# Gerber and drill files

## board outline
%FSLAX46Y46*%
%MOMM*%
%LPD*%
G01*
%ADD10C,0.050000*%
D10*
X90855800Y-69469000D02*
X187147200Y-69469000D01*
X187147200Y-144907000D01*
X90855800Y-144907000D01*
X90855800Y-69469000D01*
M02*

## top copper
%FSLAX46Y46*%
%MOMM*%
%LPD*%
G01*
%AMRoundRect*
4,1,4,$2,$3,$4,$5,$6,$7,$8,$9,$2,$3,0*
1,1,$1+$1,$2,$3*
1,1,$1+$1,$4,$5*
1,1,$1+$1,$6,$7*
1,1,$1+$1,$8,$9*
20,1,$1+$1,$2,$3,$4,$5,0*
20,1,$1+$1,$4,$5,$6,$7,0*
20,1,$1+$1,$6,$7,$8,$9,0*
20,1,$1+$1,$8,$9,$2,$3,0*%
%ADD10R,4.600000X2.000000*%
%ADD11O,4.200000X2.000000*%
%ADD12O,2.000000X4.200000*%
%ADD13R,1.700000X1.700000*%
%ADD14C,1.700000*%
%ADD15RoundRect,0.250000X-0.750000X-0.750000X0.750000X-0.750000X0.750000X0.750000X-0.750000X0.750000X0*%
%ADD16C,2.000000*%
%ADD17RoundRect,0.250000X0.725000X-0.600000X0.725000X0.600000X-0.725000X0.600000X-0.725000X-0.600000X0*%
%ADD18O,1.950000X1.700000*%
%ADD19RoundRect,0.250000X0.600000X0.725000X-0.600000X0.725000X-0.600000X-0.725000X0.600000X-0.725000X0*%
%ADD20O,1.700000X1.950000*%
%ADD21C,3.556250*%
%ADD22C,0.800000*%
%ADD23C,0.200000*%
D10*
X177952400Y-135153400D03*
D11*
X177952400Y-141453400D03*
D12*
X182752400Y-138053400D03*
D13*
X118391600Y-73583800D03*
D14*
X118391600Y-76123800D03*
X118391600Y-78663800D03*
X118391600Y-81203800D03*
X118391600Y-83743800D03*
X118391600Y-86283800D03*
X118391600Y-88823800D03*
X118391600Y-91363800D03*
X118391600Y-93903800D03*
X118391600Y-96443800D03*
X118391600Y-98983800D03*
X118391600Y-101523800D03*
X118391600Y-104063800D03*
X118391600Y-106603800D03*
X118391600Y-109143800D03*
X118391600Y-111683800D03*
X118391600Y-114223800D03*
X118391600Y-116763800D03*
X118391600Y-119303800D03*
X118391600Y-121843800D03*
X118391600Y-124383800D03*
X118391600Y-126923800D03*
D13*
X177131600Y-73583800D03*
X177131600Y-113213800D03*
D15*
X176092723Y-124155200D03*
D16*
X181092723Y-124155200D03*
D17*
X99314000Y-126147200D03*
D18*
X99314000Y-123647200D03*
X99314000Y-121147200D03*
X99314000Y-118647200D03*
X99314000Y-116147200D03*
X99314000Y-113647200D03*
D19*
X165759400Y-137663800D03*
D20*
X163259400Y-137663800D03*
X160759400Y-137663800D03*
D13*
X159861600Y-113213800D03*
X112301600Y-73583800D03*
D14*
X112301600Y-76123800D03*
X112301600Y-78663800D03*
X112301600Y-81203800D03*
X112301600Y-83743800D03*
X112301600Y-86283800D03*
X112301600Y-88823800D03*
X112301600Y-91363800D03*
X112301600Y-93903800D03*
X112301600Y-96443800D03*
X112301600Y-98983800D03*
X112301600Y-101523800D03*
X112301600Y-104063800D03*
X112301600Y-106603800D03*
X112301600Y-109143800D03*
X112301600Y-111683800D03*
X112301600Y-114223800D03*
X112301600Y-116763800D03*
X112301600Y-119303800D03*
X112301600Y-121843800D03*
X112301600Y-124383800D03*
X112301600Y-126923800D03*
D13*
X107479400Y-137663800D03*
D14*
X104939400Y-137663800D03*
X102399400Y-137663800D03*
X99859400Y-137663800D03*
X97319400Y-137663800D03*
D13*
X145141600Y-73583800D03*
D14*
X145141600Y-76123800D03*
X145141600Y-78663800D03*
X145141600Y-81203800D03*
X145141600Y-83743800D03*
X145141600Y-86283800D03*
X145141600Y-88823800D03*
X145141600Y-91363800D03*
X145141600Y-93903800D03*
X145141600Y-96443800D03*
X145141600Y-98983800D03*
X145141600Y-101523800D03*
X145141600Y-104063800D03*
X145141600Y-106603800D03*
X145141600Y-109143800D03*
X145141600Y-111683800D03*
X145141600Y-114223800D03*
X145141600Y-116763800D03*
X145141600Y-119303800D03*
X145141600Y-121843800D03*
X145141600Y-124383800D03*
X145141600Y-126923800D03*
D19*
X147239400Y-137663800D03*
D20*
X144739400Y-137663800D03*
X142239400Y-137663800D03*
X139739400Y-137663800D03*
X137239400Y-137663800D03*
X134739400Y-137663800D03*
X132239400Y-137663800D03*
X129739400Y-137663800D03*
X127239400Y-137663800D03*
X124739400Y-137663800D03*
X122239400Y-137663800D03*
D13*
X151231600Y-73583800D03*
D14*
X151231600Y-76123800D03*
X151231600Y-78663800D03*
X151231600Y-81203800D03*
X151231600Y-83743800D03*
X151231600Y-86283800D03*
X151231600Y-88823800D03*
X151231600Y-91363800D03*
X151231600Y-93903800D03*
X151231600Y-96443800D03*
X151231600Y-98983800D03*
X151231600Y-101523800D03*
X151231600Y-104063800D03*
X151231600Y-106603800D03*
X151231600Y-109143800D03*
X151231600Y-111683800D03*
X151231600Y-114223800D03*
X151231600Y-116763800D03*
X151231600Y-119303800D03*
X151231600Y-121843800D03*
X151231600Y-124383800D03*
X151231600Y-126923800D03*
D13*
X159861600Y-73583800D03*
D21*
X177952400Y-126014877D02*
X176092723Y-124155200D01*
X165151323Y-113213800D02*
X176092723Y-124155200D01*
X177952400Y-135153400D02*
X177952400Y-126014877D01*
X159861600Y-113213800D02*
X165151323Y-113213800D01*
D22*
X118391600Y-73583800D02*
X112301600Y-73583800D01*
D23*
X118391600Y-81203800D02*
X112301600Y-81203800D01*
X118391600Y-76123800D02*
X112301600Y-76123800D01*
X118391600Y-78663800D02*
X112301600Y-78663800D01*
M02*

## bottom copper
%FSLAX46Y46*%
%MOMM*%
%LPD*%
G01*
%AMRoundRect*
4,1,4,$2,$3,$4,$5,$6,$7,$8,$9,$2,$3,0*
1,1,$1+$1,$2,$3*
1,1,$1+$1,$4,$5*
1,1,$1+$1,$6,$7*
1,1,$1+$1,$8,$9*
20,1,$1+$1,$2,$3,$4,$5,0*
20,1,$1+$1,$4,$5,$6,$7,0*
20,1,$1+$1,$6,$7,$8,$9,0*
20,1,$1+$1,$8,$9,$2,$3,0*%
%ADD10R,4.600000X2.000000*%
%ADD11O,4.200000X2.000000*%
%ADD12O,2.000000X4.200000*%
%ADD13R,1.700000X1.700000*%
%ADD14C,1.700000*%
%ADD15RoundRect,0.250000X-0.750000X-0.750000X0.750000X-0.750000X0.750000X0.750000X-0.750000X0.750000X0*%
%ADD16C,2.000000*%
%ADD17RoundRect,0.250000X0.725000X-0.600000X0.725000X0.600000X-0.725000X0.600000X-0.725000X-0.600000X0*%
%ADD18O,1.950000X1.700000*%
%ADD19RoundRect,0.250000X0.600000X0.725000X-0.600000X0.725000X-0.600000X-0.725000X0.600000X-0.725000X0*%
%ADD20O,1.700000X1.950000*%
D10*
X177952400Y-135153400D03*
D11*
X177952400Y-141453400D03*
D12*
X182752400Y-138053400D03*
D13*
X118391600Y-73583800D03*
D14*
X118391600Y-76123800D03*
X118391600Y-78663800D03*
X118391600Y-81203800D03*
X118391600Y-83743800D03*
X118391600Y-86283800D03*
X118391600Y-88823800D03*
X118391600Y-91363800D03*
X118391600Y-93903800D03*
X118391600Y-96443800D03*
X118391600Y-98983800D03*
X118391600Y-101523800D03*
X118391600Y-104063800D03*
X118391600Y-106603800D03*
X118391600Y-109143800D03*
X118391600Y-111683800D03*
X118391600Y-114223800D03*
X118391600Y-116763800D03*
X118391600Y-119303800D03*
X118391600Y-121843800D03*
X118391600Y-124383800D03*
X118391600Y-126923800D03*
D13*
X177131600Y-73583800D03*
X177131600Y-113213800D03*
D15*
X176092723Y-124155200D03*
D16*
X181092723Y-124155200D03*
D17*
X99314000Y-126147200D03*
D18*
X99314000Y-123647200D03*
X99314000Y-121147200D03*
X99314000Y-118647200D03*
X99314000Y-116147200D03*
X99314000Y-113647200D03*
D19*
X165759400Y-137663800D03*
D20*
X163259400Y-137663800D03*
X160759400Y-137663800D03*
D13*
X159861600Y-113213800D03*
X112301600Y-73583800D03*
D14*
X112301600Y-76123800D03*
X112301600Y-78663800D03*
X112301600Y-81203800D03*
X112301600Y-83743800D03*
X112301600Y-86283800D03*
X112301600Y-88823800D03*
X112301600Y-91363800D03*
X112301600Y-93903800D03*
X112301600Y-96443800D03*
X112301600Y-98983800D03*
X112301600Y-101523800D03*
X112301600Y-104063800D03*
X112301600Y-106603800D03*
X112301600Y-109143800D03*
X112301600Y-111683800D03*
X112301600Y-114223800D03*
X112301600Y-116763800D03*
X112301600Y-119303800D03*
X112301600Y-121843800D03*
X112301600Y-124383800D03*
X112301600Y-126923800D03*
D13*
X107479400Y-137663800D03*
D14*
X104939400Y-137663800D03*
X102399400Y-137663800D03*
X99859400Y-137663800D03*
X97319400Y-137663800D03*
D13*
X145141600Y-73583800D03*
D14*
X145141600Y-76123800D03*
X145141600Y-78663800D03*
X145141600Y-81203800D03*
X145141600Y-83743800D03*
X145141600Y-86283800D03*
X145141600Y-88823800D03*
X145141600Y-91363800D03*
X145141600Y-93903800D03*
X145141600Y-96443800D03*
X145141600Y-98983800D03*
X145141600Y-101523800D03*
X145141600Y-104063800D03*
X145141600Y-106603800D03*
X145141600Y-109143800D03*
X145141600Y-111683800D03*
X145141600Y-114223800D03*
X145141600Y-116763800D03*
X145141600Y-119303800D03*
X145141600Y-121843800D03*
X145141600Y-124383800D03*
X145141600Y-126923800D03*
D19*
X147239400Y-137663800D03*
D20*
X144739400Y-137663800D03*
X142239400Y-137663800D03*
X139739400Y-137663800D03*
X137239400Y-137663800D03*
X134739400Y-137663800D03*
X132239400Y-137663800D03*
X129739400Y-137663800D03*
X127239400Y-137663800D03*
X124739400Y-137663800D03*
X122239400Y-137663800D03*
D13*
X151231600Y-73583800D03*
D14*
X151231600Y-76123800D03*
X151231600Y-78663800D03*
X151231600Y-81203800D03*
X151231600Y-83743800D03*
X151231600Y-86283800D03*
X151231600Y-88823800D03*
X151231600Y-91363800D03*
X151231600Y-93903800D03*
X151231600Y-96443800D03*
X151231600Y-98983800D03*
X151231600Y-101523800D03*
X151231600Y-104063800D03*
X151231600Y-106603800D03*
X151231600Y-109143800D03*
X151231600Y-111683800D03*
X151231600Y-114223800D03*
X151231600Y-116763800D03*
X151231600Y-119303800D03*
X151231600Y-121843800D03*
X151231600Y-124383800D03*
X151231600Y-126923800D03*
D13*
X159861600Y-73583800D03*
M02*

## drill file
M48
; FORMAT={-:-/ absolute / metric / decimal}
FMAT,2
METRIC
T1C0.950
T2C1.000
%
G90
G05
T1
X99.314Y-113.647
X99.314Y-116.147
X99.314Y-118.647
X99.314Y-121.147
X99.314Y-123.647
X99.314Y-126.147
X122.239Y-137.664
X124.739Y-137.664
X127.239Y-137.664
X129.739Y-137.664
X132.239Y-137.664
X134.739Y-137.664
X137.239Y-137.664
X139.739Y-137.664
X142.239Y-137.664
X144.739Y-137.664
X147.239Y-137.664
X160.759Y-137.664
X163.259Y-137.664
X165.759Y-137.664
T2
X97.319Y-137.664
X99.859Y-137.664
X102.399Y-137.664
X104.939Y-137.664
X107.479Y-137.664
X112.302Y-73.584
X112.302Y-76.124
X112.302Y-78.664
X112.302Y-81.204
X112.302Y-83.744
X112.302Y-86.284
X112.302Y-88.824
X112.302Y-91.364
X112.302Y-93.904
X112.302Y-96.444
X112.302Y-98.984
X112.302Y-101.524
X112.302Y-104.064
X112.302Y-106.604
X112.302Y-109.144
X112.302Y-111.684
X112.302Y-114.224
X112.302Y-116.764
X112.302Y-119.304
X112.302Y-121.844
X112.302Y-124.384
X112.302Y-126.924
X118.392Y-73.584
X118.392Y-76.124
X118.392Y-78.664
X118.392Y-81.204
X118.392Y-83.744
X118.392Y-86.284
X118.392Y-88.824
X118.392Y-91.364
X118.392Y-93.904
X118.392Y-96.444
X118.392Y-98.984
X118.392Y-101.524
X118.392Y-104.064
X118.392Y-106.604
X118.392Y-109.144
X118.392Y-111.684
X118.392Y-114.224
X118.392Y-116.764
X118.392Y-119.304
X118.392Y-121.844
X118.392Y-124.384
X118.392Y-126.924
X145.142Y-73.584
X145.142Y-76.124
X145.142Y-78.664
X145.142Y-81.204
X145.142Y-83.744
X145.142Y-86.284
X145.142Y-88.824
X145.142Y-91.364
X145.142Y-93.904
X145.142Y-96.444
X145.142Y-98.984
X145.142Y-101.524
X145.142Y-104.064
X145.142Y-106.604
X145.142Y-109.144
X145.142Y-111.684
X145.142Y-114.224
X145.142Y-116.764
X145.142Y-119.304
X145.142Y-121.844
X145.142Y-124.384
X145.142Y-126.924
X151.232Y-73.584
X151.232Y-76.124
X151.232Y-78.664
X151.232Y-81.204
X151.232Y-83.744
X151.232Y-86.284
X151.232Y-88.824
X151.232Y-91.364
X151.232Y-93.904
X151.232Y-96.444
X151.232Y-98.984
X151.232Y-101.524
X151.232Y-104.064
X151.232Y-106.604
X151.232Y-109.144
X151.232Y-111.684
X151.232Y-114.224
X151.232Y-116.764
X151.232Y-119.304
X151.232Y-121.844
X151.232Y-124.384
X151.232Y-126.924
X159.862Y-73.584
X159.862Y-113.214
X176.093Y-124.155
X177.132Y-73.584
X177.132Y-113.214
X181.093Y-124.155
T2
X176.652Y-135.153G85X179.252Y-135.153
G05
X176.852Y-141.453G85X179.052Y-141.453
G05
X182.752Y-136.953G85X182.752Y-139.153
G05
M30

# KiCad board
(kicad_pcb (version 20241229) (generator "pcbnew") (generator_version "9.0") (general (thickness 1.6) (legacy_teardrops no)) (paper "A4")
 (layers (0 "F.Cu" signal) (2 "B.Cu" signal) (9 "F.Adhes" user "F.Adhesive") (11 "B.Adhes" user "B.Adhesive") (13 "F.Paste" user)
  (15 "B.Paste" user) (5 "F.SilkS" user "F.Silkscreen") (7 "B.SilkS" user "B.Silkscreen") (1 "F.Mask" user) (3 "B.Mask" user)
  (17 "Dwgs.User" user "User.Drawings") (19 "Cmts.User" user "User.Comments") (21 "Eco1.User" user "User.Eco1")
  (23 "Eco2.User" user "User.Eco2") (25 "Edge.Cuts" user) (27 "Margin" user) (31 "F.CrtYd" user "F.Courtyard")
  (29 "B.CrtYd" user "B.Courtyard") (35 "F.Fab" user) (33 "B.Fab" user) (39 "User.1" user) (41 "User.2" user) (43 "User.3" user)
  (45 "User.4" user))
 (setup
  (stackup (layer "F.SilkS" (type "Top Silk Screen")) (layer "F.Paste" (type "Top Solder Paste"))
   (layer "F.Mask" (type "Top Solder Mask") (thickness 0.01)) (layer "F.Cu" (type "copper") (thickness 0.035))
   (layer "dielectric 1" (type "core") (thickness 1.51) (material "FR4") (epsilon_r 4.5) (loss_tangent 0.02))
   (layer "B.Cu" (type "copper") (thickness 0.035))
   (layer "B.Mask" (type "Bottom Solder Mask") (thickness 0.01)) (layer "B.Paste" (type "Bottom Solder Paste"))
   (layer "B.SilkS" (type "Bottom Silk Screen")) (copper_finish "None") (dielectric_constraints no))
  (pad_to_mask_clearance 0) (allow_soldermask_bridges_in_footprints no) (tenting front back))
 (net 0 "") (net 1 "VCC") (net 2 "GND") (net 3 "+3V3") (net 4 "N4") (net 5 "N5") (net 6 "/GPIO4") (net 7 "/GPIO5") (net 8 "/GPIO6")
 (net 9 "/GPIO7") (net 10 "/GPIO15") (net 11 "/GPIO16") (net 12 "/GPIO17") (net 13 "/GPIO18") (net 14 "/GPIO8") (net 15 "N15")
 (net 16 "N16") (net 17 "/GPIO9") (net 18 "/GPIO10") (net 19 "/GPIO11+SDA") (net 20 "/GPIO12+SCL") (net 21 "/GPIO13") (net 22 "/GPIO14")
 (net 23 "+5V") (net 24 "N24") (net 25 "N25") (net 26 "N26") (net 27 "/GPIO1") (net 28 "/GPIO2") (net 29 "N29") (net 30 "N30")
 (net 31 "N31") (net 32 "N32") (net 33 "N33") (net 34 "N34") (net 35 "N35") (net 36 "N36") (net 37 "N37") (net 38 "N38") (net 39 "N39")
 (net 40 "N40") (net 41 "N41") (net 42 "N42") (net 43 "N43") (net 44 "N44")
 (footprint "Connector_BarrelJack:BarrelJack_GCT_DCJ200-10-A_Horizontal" (layer "F.Cu") (at 177.9524 135.1534)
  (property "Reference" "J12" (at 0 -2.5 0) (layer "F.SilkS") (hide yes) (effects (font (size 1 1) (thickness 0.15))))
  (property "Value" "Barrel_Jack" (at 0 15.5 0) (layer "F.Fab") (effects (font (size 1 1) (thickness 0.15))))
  (pad "1" thru_hole rect (at 0 0) (size 4.6 2) (drill oval 3.6 1) (layers "*.Cu" "*.Mask") (remove_unused_layers no) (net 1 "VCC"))
  (pad "2" thru_hole oval (at 0 6.3) (size 4.2 2) (drill oval 3.2 1) (layers "*.Cu" "*.Mask") (remove_unused_layers no) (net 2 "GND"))
  (pad "3" thru_hole oval (at 4.8 2.9) (size 2 4.2) (drill oval 1 3.2) (layers "*.Cu" "*.Mask") (remove_unused_layers no)))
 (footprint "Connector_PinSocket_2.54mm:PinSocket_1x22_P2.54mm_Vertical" (layer "F.Cu") (at 118.3916 73.5838)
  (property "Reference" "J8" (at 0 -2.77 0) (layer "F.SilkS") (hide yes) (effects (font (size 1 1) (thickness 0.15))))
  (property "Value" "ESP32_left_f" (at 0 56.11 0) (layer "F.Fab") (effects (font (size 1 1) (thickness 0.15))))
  (pad "1" thru_hole rect (at 0 0) (size 1.7 1.7) (drill 1) (layers "*.Cu" "*.Mask") (remove_unused_layers no) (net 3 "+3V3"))
  (pad "2" thru_hole circle (at 0 2.54) (size 1.7 1.7) (drill 1) (layers "*.Cu" "*.Mask") (remove_unused_layers no) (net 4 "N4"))
  (pad "3" thru_hole circle (at 0 5.08) (size 1.7 1.7) (drill 1) (layers "*.Cu" "*.Mask") (remove_unused_layers no) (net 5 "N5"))
  (pad "4" thru_hole circle (at 0 7.62) (size 1.7 1.7) (drill 1) (layers "*.Cu" "*.Mask") (remove_unused_layers no) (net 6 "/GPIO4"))
  (pad "5" thru_hole circle (at 0 10.16) (size 1.7 1.7) (drill 1) (layers "*.Cu" "*.Mask") (remove_unused_layers no) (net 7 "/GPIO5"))
  (pad "6" thru_hole circle (at 0 12.7) (size 1.7 1.7) (drill 1) (layers "*.Cu" "*.Mask") (remove_unused_layers no) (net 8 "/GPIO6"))
  (pad "7" thru_hole circle (at 0 15.24) (size 1.7 1.7) (drill 1) (layers "*.Cu" "*.Mask") (remove_unused_layers no) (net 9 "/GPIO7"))
  (pad "8" thru_hole circle (at 0 17.78) (size 1.7 1.7) (drill 1) (layers "*.Cu" "*.Mask") (remove_unused_layers no) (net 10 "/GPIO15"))
  (pad "9" thru_hole circle (at 0 20.32) (size 1.7 1.7) (drill 1) (layers "*.Cu" "*.Mask") (remove_unused_layers no) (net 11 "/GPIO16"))
  (pad "10" thru_hole circle (at 0 22.86) (size 1.7 1.7) (drill 1) (layers "*.Cu" "*.Mask") (remove_unused_layers no) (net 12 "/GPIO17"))
  (pad "11" thru_hole circle (at 0 25.4) (size 1.7 1.7) (drill 1) (layers "*.Cu" "*.Mask") (remove_unused_layers no) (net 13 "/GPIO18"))
  (pad "12" thru_hole circle (at 0 27.94) (size 1.7 1.7) (drill 1) (layers "*.Cu" "*.Mask") (remove_unused_layers no) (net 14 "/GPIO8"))
  (pad "13" thru_hole circle (at 0 30.48) (size 1.7 1.7) (drill 1) (layers "*.Cu" "*.Mask") (remove_unused_layers no) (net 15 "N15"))
  (pad "14" thru_hole circle (at 0 33.02) (size 1.7 1.7) (drill 1) (layers "*.Cu" "*.Mask") (remove_unused_layers no) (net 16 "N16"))
  (pad "15" thru_hole circle (at 0 35.56) (size 1.7 1.7) (drill 1) (layers "*.Cu" "*.Mask") (remove_unused_layers no) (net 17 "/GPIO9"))
  (pad "16" thru_hole circle (at 0 38.1) (size 1.7 1.7) (drill 1) (layers "*.Cu" "*.Mask") (remove_unused_layers no) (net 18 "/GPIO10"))
  (pad "17" thru_hole circle (at 0 40.64) (size 1.7 1.7) (drill 1) (layers "*.Cu" "*.Mask") (remove_unused_layers no) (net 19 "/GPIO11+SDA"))
  (pad "18" thru_hole circle (at 0 43.18) (size 1.7 1.7) (drill 1) (layers "*.Cu" "*.Mask") (remove_unused_layers no) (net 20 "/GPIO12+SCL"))
  (pad "19" thru_hole circle (at 0 45.72) (size 1.7 1.7) (drill 1) (layers "*.Cu" "*.Mask") (remove_unused_layers no) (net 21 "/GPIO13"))
  (pad "20" thru_hole circle (at 0 48.26) (size 1.7 1.7) (drill 1) (layers "*.Cu" "*.Mask") (remove_unused_layers no) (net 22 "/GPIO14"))
  (pad "21" thru_hole circle (at 0 50.8) (size 1.7 1.7) (drill 1) (layers "*.Cu" "*.Mask") (remove_unused_layers no) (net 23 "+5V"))
  (pad "22" thru_hole circle (at 0 53.34) (size 1.7 1.7) (drill 1) (layers "*.Cu" "*.Mask") (remove_unused_layers no) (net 2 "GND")))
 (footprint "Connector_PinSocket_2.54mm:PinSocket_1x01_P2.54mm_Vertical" (layer "F.Cu") (at 177.1316 73.5838)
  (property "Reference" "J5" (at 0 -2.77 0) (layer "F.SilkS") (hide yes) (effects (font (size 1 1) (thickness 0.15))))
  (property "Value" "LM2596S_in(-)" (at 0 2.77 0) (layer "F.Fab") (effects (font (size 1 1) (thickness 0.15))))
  (pad "1" thru_hole rect (at 0 0) (size 1.7 1.7) (drill 1) (layers "*.Cu" "*.Mask") (remove_unused_layers no) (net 2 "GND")))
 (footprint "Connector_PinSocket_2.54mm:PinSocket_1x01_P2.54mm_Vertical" (layer "F.Cu") (at 177.1316 113.2138)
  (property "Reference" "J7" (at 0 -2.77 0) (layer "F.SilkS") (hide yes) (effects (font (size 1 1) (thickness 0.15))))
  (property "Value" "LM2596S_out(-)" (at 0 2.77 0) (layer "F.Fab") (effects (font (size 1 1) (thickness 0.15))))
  (pad "1" thru_hole rect (at 0 0) (size 1.7 1.7) (drill 1) (layers "*.Cu" "*.Mask") (remove_unused_layers no) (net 2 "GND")))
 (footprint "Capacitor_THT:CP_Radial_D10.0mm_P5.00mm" (layer "F.Cu") (at 176.092723 124.1552)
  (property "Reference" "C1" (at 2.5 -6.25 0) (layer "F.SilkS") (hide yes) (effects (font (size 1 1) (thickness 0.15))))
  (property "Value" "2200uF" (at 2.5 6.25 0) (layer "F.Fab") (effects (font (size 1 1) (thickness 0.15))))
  (pad "1" thru_hole roundrect (at 0 0) (size 2 2) (drill 1) (layers "*.Cu" "*.Mask") (remove_unused_layers no) (roundrect_rratio 0.125)
   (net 1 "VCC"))
  (pad "2" thru_hole circle (at 5 0) (size 2 2) (drill 1) (layers "*.Cu" "*.Mask") (remove_unused_layers no) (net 2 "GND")))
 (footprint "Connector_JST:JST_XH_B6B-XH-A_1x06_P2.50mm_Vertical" (layer "F.Cu") (at 99.314 126.1472 90)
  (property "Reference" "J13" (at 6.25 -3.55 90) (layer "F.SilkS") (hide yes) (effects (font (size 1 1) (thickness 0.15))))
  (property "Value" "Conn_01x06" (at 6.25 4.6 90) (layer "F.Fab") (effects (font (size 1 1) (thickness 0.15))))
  (pad "1" thru_hole roundrect (at 0 0 90) (size 1.7 1.95) (drill 0.95) (layers "*.Cu" "*.Mask") (remove_unused_layers no)
   (roundrect_rratio 0.147059) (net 12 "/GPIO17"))
  (pad "2" thru_hole oval (at 2.5 0 90) (size 1.7 1.95) (drill 0.95) (layers "*.Cu" "*.Mask") (remove_unused_layers no) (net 2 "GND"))
  (pad "3" thru_hole oval (at 5 0 90) (size 1.7 1.95) (drill 0.95) (layers "*.Cu" "*.Mask") (remove_unused_layers no) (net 21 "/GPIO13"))
  (pad "4" thru_hole oval (at 7.5 0 90) (size 1.7 1.95) (drill 0.95) (layers "*.Cu" "*.Mask") (remove_unused_layers no) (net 22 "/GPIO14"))
  (pad "5" thru_hole oval (at 10 0 90) (size 1.7 1.95) (drill 0.95) (layers "*.Cu" "*.Mask") (remove_unused_layers no) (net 3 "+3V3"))
  (pad "6" thru_hole oval (at 12.5 0 90) (size 1.7 1.95) (drill 0.95) (layers "*.Cu" "*.Mask") (remove_unused_layers no) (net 13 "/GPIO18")))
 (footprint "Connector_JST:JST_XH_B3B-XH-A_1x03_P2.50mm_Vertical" (layer "F.Cu") (at 165.7594 137.6638 180)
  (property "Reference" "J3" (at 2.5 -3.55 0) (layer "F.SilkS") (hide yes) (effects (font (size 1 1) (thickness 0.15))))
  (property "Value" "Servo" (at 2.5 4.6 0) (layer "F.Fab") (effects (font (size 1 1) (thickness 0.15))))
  (pad "1" thru_hole roundrect (at 0 0 180) (size 1.7 1.95) (drill 0.95) (layers "*.Cu" "*.Mask") (remove_unused_layers no)
   (roundrect_rratio 0.147059) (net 10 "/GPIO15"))
  (pad "2" thru_hole oval (at 2.5 0 180) (size 1.7 1.95) (drill 0.95) (layers "*.Cu" "*.Mask") (remove_unused_layers no) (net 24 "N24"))
  (pad "3" thru_hole oval (at 5 0 180) (size 1.7 1.95) (drill 0.95) (layers "*.Cu" "*.Mask") (remove_unused_layers no) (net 2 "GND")))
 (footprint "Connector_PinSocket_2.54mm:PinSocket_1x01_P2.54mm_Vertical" (layer "F.Cu") (at 159.8616 113.2138)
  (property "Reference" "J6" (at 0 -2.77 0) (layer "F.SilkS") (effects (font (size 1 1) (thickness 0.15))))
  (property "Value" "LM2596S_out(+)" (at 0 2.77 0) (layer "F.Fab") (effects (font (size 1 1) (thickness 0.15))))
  (pad "1" thru_hole rect (at 0 0) (size 1.7 1.7) (drill 1) (layers "*.Cu" "*.Mask") (remove_unused_layers no) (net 1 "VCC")))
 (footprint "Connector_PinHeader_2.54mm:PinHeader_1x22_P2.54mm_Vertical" (layer "F.Cu") (at 112.3016 73.5838)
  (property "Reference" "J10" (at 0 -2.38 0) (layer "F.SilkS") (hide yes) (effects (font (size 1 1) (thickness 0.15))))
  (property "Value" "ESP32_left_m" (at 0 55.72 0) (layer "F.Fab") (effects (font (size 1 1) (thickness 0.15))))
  (pad "1" thru_hole rect (at 0 0) (size 1.7 1.7) (drill 1) (layers "*.Cu" "*.Mask") (remove_unused_layers no) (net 3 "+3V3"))
  (pad "2" thru_hole circle (at 0 2.54) (size 1.7 1.7) (drill 1) (layers "*.Cu" "*.Mask") (remove_unused_layers no) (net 4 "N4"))
  (pad "3" thru_hole circle (at 0 5.08) (size 1.7 1.7) (drill 1) (layers "*.Cu" "*.Mask") (remove_unused_layers no) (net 5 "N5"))
  (pad "4" thru_hole circle (at 0 7.62) (size 1.7 1.7) (drill 1) (layers "*.Cu" "*.Mask") (remove_unused_layers no) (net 6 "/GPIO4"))
  (pad "5" thru_hole circle (at 0 10.16) (size 1.7 1.7) (drill 1) (layers "*.Cu" "*.Mask") (remove_unused_layers no) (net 7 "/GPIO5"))
  (pad "6" thru_hole circle (at 0 12.7) (size 1.7 1.7) (drill 1) (layers "*.Cu" "*.Mask") (remove_unused_layers no) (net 8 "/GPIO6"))
  (pad "7" thru_hole circle (at 0 15.24) (size 1.7 1.7) (drill 1) (layers "*.Cu" "*.Mask") (remove_unused_layers no) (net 9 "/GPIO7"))
  (pad "8" thru_hole circle (at 0 17.78) (size 1.7 1.7) (drill 1) (layers "*.Cu" "*.Mask") (remove_unused_layers no) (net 10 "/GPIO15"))
  (pad "9" thru_hole circle (at 0 20.32) (size 1.7 1.7) (drill 1) (layers "*.Cu" "*.Mask") (remove_unused_layers no) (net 11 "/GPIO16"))
  (pad "10" thru_hole circle (at 0 22.86) (size 1.7 1.7) (drill 1) (layers "*.Cu" "*.Mask") (remove_unused_layers no) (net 12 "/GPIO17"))
  (pad "11" thru_hole circle (at 0 25.4) (size 1.7 1.7) (drill 1) (layers "*.Cu" "*.Mask") (remove_unused_layers no) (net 13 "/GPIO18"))
  (pad "12" thru_hole circle (at 0 27.94) (size 1.7 1.7) (drill 1) (layers "*.Cu" "*.Mask") (remove_unused_layers no) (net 14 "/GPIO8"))
  (pad "13" thru_hole circle (at 0 30.48) (size 1.7 1.7) (drill 1) (layers "*.Cu" "*.Mask") (remove_unused_layers no) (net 15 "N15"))
  (pad "14" thru_hole circle (at 0 33.02) (size 1.7 1.7) (drill 1) (layers "*.Cu" "*.Mask") (remove_unused_layers no) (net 16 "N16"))
  (pad "15" thru_hole circle (at 0 35.56) (size 1.7 1.7) (drill 1) (layers "*.Cu" "*.Mask") (remove_unused_layers no) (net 17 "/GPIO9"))
  (pad "16" thru_hole circle (at 0 38.1) (size 1.7 1.7) (drill 1) (layers "*.Cu" "*.Mask") (remove_unused_layers no) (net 18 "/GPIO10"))
  (pad "17" thru_hole circle (at 0 40.64) (size 1.7 1.7) (drill 1) (layers "*.Cu" "*.Mask") (remove_unused_layers no) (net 19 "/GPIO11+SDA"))
  (pad "18" thru_hole circle (at 0 43.18) (size 1.7 1.7) (drill 1) (layers "*.Cu" "*.Mask") (remove_unused_layers no) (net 20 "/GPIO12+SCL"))
  (pad "19" thru_hole circle (at 0 45.72) (size 1.7 1.7) (drill 1) (layers "*.Cu" "*.Mask") (remove_unused_layers no) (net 21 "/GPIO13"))
  (pad "20" thru_hole circle (at 0 48.26) (size 1.7 1.7) (drill 1) (layers "*.Cu" "*.Mask") (remove_unused_layers no) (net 22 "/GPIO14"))
  (pad "21" thru_hole circle (at 0 50.8) (size 1.7 1.7) (drill 1) (layers "*.Cu" "*.Mask") (remove_unused_layers no) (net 23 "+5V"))
  (pad "22" thru_hole circle (at 0 53.34) (size 1.7 1.7) (drill 1) (layers "*.Cu" "*.Mask") (remove_unused_layers no) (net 2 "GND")))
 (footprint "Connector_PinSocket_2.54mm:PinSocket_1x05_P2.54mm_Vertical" (layer "F.Cu") (at 107.4794 137.6638 -90)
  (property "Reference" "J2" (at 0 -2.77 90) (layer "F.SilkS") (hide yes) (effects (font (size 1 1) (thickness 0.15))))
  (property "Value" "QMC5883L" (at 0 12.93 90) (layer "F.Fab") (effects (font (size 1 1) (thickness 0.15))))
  (pad "1" thru_hole rect (at 0 0 270) (size 1.7 1.7) (drill 1) (layers "*.Cu" "*.Mask") (remove_unused_layers no) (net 3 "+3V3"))
  (pad "2" thru_hole circle (at 0 2.54 270) (size 1.7 1.7) (drill 1) (layers "*.Cu" "*.Mask") (remove_unused_layers no) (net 2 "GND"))
  (pad "3" thru_hole circle (at 0 5.08 270) (size 1.7 1.7) (drill 1) (layers "*.Cu" "*.Mask") (remove_unused_layers no)
   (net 20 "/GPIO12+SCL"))
  (pad "4" thru_hole circle (at 0 7.62 270) (size 1.7 1.7) (drill 1) (layers "*.Cu" "*.Mask") (remove_unused_layers no)
   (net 19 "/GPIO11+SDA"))
  (pad "5" thru_hole circle (at 0 10.16 270) (size 1.7 1.7) (drill 1) (layers "*.Cu" "*.Mask") (remove_unused_layers no) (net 11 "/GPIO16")))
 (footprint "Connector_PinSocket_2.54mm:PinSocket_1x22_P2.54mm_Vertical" (layer "F.Cu") (at 145.1416 73.5838)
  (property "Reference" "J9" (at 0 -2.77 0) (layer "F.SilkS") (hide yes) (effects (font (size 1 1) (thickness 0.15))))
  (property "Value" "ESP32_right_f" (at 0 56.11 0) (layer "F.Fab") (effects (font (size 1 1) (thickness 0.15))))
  (pad "1" thru_hole rect (at 0 0) (size 1.7 1.7) (drill 1) (layers "*.Cu" "*.Mask") (remove_unused_layers no) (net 2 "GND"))
  (pad "2" thru_hole circle (at 0 2.54) (size 1.7 1.7) (drill 1) (layers "*.Cu" "*.Mask") (remove_unused_layers no) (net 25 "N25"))
  (pad "3" thru_hole circle (at 0 5.08) (size 1.7 1.7) (drill 1) (layers "*.Cu" "*.Mask") (remove_unused_layers no) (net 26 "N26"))
  (pad "4" thru_hole circle (at 0 7.62) (size 1.7 1.7) (drill 1) (layers "*.Cu" "*.Mask") (remove_unused_layers no) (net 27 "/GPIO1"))
  (pad "5" thru_hole circle (at 0 10.16) (size 1.7 1.7) (drill 1) (layers "*.Cu" "*.Mask") (remove_unused_layers no) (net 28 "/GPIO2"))
  (pad "6" thru_hole circle (at 0 12.7) (size 1.7 1.7) (drill 1) (layers "*.Cu" "*.Mask") (remove_unused_layers no) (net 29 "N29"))
  (pad "7" thru_hole circle (at 0 15.24) (size 1.7 1.7) (drill 1) (layers "*.Cu" "*.Mask") (remove_unused_layers no) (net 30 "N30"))
  (pad "8" thru_hole circle (at 0 17.78) (size 1.7 1.7) (drill 1) (layers "*.Cu" "*.Mask") (remove_unused_layers no) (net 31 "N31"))
  (pad "9" thru_hole circle (at 0 20.32) (size 1.7 1.7) (drill 1) (layers "*.Cu" "*.Mask") (remove_unused_layers no) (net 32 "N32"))
  (pad "10" thru_hole circle (at 0 22.86) (size 1.7 1.7) (drill 1) (layers "*.Cu" "*.Mask") (remove_unused_layers no) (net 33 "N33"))
  (pad "11" thru_hole circle (at 0 25.4) (size 1.7 1.7) (drill 1) (layers "*.Cu" "*.Mask") (remove_unused_layers no) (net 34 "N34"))
  (pad "12" thru_hole circle (at 0 27.94) (size 1.7 1.7) (drill 1) (layers "*.Cu" "*.Mask") (remove_unused_layers no) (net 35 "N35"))
  (pad "13" thru_hole circle (at 0 30.48) (size 1.7 1.7) (drill 1) (layers "*.Cu" "*.Mask") (remove_unused_layers no) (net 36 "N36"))
  (pad "14" thru_hole circle (at 0 33.02) (size 1.7 1.7) (drill 1) (layers "*.Cu" "*.Mask") (remove_unused_layers no) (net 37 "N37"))
  (pad "15" thru_hole circle (at 0 35.56) (size 1.7 1.7) (drill 1) (layers "*.Cu" "*.Mask") (remove_unused_layers no) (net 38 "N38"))
  (pad "16" thru_hole circle (at 0 38.1) (size 1.7 1.7) (drill 1) (layers "*.Cu" "*.Mask") (remove_unused_layers no) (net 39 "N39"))
  (pad "17" thru_hole circle (at 0 40.64) (size 1.7 1.7) (drill 1) (layers "*.Cu" "*.Mask") (remove_unused_layers no) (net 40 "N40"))
  (pad "18" thru_hole circle (at 0 43.18) (size 1.7 1.7) (drill 1) (layers "*.Cu" "*.Mask") (remove_unused_layers no) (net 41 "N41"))
  (pad "19" thru_hole circle (at 0 45.72) (size 1.7 1.7) (drill 1) (layers "*.Cu" "*.Mask") (remove_unused_layers no) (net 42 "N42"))
  (pad "20" thru_hole circle (at 0 48.26) (size 1.7 1.7) (drill 1) (layers "*.Cu" "*.Mask") (remove_unused_layers no) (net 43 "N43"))
  (pad "21" thru_hole circle (at 0 50.8) (size 1.7 1.7) (drill 1) (layers "*.Cu" "*.Mask") (remove_unused_layers no) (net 2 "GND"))
  (pad "22" thru_hole circle (at 0 53.34) (size 1.7 1.7) (drill 1) (layers "*.Cu" "*.Mask") (remove_unused_layers no) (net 2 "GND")))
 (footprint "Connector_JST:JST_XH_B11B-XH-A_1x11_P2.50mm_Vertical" (layer "F.Cu") (at 147.2394 137.6638 180)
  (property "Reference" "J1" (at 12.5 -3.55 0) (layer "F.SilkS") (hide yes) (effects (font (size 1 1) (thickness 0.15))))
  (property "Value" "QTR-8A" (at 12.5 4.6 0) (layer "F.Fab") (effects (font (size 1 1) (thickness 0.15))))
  (pad "1" thru_hole roundrect (at 0 0 180) (size 1.7 1.95) (drill 0.95) (layers "*.Cu" "*.Mask") (remove_unused_layers no)
   (roundrect_rratio 0.147059) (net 6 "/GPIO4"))
  (pad "2" thru_hole oval (at 2.5 0 180) (size 1.7 1.95) (drill 0.95) (layers "*.Cu" "*.Mask") (remove_unused_layers no) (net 7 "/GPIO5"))
  (pad "3" thru_hole oval (at 5 0 180) (size 1.7 1.95) (drill 0.95) (layers "*.Cu" "*.Mask") (remove_unused_layers no) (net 8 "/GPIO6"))
  (pad "4" thru_hole oval (at 7.5 0 180) (size 1.7 1.95) (drill 0.95) (layers "*.Cu" "*.Mask") (remove_unused_layers no) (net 9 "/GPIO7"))
  (pad "5" thru_hole oval (at 10 0 180) (size 1.7 1.95) (drill 0.95) (layers "*.Cu" "*.Mask") (remove_unused_layers no) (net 14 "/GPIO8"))
  (pad "6" thru_hole oval (at 12.5 0 180) (size 1.7 1.95) (drill 0.95) (layers "*.Cu" "*.Mask") (remove_unused_layers no) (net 17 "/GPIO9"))
  (pad "7" thru_hole oval (at 15 0 180) (size 1.7 1.95) (drill 0.95) (layers "*.Cu" "*.Mask") (remove_unused_layers no) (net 18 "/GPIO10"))
  (pad "8" thru_hole oval (at 17.5 0 180) (size 1.7 1.95) (drill 0.95) (layers "*.Cu" "*.Mask") (remove_unused_layers no) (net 27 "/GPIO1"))
  (pad "9" thru_hole oval (at 20 0 180) (size 1.7 1.95) (drill 0.95) (layers "*.Cu" "*.Mask") (remove_unused_layers no) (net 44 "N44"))
  (pad "10" thru_hole oval (at 22.5 0 180) (size 1.7 1.95) (drill 0.95) (layers "*.Cu" "*.Mask") (remove_unused_layers no) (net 3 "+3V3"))
  (pad "11" thru_hole oval (at 25 0 180) (size 1.7 1.95) (drill 0.95) (layers "*.Cu" "*.Mask") (remove_unused_layers no) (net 2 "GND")))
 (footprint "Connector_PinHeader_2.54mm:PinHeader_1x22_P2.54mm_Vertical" (layer "F.Cu") (at 151.2316 73.5838)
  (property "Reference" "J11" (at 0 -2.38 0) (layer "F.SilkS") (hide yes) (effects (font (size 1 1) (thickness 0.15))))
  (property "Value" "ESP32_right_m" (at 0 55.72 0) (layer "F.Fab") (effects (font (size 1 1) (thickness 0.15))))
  (pad "1" thru_hole rect (at 0 0) (size 1.7 1.7) (drill 1) (layers "*.Cu" "*.Mask") (remove_unused_layers no) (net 2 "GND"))
  (pad "2" thru_hole circle (at 0 2.54) (size 1.7 1.7) (drill 1) (layers "*.Cu" "*.Mask") (remove_unused_layers no) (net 25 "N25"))
  (pad "3" thru_hole circle (at 0 5.08) (size 1.7 1.7) (drill 1) (layers "*.Cu" "*.Mask") (remove_unused_layers no) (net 26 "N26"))
  (pad "4" thru_hole circle (at 0 7.62) (size 1.7 1.7) (drill 1) (layers "*.Cu" "*.Mask") (remove_unused_layers no) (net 27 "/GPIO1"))
  (pad "5" thru_hole circle (at 0 10.16) (size 1.7 1.7) (drill 1) (layers "*.Cu" "*.Mask") (remove_unused_layers no) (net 28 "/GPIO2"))
  (pad "6" thru_hole circle (at 0 12.7) (size 1.7 1.7) (drill 1) (layers "*.Cu" "*.Mask") (remove_unused_layers no) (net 29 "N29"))
  (pad "7" thru_hole circle (at 0 15.24) (size 1.7 1.7) (drill 1) (layers "*.Cu" "*.Mask") (remove_unused_layers no) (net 30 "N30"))
  (pad "8" thru_hole circle (at 0 17.78) (size 1.7 1.7) (drill 1) (layers "*.Cu" "*.Mask") (remove_unused_layers no) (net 31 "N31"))
  (pad "9" thru_hole circle (at 0 20.32) (size 1.7 1.7) (drill 1) (layers "*.Cu" "*.Mask") (remove_unused_layers no) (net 32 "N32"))
  (pad "10" thru_hole circle (at 0 22.86) (size 1.7 1.7) (drill 1) (layers "*.Cu" "*.Mask") (remove_unused_layers no) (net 33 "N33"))
  (pad "11" thru_hole circle (at 0 25.4) (size 1.7 1.7) (drill 1) (layers "*.Cu" "*.Mask") (remove_unused_layers no) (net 34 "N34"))
  (pad "12" thru_hole circle (at 0 27.94) (size 1.7 1.7) (drill 1) (layers "*.Cu" "*.Mask") (remove_unused_layers no) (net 35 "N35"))
  (pad "13" thru_hole circle (at 0 30.48) (size 1.7 1.7) (drill 1) (layers "*.Cu" "*.Mask") (remove_unused_layers no) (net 36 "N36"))
  (pad "14" thru_hole circle (at 0 33.02) (size 1.7 1.7) (drill 1) (layers "*.Cu" "*.Mask") (remove_unused_layers no) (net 37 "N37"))
  (pad "15" thru_hole circle (at 0 35.56) (size 1.7 1.7) (drill 1) (layers "*.Cu" "*.Mask") (remove_unused_layers no) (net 38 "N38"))
  (pad "16" thru_hole circle (at 0 38.1) (size 1.7 1.7) (drill 1) (layers "*.Cu" "*.Mask") (remove_unused_layers no) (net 39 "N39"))
  (pad "17" thru_hole circle (at 0 40.64) (size 1.7 1.7) (drill 1) (layers "*.Cu" "*.Mask") (remove_unused_layers no) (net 40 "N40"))
  (pad "18" thru_hole circle (at 0 43.18) (size 1.7 1.7) (drill 1) (layers "*.Cu" "*.Mask") (remove_unused_layers no) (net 41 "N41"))
  (pad "19" thru_hole circle (at 0 45.72) (size 1.7 1.7) (drill 1) (layers "*.Cu" "*.Mask") (remove_unused_layers no) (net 42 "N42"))
  (pad "20" thru_hole circle (at 0 48.26) (size 1.7 1.7) (drill 1) (layers "*.Cu" "*.Mask") (remove_unused_layers no) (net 43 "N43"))
  (pad "21" thru_hole circle (at 0 50.8) (size 1.7 1.7) (drill 1) (layers "*.Cu" "*.Mask") (remove_unused_layers no) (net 2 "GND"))
  (pad "22" thru_hole circle (at 0 53.34) (size 1.7 1.7) (drill 1) (layers "*.Cu" "*.Mask") (remove_unused_layers no) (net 2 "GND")))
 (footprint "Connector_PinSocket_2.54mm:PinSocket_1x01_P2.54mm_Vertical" (layer "F.Cu") (at 159.8616 73.5838)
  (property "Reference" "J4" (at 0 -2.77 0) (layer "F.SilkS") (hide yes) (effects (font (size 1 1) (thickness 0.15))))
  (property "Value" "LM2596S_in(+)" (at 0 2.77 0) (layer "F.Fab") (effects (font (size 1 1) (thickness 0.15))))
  (pad "1" thru_hole rect (at 0 0) (size 1.7 1.7) (drill 1) (layers "*.Cu" "*.Mask") (remove_unused_layers no) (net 24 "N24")))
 (gr_rect (start 90.8558 69.469) (end 187.1472 144.907) (stroke (width 0.05) (type default)) (fill no) (layer "Edge.Cuts"))
 (segment (start 177.9524 126.014877) (end 176.092723 124.1552) (width 3.55625) (layer "F.Cu") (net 1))
 (segment (start 165.151323 113.2138) (end 176.092723 124.1552) (width 3.55625) (layer "F.Cu") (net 1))
 (segment (start 177.9524 135.1534) (end 177.9524 126.014877) (width 3.55625) (layer "F.Cu") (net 1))
 (segment (start 159.8616 113.2138) (end 165.151323 113.2138) (width 3.55625) (layer "F.Cu") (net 1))
 (segment (start 118.3916 73.5838) (end 112.3016 73.5838) (width 0.8) (layer "F.Cu") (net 3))
 (segment (start 118.3916 81.2038) (end 112.3016 81.2038) (width 0.2) (layer "F.Cu") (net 6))
 (segment (start 118.3916 76.1238) (end 112.3016 76.1238) (width 0.2) (layer "F.Cu") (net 4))
 (segment (start 118.3916 78.6638) (end 112.3016 78.6638) (width 0.2) (layer "F.Cu") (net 5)))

